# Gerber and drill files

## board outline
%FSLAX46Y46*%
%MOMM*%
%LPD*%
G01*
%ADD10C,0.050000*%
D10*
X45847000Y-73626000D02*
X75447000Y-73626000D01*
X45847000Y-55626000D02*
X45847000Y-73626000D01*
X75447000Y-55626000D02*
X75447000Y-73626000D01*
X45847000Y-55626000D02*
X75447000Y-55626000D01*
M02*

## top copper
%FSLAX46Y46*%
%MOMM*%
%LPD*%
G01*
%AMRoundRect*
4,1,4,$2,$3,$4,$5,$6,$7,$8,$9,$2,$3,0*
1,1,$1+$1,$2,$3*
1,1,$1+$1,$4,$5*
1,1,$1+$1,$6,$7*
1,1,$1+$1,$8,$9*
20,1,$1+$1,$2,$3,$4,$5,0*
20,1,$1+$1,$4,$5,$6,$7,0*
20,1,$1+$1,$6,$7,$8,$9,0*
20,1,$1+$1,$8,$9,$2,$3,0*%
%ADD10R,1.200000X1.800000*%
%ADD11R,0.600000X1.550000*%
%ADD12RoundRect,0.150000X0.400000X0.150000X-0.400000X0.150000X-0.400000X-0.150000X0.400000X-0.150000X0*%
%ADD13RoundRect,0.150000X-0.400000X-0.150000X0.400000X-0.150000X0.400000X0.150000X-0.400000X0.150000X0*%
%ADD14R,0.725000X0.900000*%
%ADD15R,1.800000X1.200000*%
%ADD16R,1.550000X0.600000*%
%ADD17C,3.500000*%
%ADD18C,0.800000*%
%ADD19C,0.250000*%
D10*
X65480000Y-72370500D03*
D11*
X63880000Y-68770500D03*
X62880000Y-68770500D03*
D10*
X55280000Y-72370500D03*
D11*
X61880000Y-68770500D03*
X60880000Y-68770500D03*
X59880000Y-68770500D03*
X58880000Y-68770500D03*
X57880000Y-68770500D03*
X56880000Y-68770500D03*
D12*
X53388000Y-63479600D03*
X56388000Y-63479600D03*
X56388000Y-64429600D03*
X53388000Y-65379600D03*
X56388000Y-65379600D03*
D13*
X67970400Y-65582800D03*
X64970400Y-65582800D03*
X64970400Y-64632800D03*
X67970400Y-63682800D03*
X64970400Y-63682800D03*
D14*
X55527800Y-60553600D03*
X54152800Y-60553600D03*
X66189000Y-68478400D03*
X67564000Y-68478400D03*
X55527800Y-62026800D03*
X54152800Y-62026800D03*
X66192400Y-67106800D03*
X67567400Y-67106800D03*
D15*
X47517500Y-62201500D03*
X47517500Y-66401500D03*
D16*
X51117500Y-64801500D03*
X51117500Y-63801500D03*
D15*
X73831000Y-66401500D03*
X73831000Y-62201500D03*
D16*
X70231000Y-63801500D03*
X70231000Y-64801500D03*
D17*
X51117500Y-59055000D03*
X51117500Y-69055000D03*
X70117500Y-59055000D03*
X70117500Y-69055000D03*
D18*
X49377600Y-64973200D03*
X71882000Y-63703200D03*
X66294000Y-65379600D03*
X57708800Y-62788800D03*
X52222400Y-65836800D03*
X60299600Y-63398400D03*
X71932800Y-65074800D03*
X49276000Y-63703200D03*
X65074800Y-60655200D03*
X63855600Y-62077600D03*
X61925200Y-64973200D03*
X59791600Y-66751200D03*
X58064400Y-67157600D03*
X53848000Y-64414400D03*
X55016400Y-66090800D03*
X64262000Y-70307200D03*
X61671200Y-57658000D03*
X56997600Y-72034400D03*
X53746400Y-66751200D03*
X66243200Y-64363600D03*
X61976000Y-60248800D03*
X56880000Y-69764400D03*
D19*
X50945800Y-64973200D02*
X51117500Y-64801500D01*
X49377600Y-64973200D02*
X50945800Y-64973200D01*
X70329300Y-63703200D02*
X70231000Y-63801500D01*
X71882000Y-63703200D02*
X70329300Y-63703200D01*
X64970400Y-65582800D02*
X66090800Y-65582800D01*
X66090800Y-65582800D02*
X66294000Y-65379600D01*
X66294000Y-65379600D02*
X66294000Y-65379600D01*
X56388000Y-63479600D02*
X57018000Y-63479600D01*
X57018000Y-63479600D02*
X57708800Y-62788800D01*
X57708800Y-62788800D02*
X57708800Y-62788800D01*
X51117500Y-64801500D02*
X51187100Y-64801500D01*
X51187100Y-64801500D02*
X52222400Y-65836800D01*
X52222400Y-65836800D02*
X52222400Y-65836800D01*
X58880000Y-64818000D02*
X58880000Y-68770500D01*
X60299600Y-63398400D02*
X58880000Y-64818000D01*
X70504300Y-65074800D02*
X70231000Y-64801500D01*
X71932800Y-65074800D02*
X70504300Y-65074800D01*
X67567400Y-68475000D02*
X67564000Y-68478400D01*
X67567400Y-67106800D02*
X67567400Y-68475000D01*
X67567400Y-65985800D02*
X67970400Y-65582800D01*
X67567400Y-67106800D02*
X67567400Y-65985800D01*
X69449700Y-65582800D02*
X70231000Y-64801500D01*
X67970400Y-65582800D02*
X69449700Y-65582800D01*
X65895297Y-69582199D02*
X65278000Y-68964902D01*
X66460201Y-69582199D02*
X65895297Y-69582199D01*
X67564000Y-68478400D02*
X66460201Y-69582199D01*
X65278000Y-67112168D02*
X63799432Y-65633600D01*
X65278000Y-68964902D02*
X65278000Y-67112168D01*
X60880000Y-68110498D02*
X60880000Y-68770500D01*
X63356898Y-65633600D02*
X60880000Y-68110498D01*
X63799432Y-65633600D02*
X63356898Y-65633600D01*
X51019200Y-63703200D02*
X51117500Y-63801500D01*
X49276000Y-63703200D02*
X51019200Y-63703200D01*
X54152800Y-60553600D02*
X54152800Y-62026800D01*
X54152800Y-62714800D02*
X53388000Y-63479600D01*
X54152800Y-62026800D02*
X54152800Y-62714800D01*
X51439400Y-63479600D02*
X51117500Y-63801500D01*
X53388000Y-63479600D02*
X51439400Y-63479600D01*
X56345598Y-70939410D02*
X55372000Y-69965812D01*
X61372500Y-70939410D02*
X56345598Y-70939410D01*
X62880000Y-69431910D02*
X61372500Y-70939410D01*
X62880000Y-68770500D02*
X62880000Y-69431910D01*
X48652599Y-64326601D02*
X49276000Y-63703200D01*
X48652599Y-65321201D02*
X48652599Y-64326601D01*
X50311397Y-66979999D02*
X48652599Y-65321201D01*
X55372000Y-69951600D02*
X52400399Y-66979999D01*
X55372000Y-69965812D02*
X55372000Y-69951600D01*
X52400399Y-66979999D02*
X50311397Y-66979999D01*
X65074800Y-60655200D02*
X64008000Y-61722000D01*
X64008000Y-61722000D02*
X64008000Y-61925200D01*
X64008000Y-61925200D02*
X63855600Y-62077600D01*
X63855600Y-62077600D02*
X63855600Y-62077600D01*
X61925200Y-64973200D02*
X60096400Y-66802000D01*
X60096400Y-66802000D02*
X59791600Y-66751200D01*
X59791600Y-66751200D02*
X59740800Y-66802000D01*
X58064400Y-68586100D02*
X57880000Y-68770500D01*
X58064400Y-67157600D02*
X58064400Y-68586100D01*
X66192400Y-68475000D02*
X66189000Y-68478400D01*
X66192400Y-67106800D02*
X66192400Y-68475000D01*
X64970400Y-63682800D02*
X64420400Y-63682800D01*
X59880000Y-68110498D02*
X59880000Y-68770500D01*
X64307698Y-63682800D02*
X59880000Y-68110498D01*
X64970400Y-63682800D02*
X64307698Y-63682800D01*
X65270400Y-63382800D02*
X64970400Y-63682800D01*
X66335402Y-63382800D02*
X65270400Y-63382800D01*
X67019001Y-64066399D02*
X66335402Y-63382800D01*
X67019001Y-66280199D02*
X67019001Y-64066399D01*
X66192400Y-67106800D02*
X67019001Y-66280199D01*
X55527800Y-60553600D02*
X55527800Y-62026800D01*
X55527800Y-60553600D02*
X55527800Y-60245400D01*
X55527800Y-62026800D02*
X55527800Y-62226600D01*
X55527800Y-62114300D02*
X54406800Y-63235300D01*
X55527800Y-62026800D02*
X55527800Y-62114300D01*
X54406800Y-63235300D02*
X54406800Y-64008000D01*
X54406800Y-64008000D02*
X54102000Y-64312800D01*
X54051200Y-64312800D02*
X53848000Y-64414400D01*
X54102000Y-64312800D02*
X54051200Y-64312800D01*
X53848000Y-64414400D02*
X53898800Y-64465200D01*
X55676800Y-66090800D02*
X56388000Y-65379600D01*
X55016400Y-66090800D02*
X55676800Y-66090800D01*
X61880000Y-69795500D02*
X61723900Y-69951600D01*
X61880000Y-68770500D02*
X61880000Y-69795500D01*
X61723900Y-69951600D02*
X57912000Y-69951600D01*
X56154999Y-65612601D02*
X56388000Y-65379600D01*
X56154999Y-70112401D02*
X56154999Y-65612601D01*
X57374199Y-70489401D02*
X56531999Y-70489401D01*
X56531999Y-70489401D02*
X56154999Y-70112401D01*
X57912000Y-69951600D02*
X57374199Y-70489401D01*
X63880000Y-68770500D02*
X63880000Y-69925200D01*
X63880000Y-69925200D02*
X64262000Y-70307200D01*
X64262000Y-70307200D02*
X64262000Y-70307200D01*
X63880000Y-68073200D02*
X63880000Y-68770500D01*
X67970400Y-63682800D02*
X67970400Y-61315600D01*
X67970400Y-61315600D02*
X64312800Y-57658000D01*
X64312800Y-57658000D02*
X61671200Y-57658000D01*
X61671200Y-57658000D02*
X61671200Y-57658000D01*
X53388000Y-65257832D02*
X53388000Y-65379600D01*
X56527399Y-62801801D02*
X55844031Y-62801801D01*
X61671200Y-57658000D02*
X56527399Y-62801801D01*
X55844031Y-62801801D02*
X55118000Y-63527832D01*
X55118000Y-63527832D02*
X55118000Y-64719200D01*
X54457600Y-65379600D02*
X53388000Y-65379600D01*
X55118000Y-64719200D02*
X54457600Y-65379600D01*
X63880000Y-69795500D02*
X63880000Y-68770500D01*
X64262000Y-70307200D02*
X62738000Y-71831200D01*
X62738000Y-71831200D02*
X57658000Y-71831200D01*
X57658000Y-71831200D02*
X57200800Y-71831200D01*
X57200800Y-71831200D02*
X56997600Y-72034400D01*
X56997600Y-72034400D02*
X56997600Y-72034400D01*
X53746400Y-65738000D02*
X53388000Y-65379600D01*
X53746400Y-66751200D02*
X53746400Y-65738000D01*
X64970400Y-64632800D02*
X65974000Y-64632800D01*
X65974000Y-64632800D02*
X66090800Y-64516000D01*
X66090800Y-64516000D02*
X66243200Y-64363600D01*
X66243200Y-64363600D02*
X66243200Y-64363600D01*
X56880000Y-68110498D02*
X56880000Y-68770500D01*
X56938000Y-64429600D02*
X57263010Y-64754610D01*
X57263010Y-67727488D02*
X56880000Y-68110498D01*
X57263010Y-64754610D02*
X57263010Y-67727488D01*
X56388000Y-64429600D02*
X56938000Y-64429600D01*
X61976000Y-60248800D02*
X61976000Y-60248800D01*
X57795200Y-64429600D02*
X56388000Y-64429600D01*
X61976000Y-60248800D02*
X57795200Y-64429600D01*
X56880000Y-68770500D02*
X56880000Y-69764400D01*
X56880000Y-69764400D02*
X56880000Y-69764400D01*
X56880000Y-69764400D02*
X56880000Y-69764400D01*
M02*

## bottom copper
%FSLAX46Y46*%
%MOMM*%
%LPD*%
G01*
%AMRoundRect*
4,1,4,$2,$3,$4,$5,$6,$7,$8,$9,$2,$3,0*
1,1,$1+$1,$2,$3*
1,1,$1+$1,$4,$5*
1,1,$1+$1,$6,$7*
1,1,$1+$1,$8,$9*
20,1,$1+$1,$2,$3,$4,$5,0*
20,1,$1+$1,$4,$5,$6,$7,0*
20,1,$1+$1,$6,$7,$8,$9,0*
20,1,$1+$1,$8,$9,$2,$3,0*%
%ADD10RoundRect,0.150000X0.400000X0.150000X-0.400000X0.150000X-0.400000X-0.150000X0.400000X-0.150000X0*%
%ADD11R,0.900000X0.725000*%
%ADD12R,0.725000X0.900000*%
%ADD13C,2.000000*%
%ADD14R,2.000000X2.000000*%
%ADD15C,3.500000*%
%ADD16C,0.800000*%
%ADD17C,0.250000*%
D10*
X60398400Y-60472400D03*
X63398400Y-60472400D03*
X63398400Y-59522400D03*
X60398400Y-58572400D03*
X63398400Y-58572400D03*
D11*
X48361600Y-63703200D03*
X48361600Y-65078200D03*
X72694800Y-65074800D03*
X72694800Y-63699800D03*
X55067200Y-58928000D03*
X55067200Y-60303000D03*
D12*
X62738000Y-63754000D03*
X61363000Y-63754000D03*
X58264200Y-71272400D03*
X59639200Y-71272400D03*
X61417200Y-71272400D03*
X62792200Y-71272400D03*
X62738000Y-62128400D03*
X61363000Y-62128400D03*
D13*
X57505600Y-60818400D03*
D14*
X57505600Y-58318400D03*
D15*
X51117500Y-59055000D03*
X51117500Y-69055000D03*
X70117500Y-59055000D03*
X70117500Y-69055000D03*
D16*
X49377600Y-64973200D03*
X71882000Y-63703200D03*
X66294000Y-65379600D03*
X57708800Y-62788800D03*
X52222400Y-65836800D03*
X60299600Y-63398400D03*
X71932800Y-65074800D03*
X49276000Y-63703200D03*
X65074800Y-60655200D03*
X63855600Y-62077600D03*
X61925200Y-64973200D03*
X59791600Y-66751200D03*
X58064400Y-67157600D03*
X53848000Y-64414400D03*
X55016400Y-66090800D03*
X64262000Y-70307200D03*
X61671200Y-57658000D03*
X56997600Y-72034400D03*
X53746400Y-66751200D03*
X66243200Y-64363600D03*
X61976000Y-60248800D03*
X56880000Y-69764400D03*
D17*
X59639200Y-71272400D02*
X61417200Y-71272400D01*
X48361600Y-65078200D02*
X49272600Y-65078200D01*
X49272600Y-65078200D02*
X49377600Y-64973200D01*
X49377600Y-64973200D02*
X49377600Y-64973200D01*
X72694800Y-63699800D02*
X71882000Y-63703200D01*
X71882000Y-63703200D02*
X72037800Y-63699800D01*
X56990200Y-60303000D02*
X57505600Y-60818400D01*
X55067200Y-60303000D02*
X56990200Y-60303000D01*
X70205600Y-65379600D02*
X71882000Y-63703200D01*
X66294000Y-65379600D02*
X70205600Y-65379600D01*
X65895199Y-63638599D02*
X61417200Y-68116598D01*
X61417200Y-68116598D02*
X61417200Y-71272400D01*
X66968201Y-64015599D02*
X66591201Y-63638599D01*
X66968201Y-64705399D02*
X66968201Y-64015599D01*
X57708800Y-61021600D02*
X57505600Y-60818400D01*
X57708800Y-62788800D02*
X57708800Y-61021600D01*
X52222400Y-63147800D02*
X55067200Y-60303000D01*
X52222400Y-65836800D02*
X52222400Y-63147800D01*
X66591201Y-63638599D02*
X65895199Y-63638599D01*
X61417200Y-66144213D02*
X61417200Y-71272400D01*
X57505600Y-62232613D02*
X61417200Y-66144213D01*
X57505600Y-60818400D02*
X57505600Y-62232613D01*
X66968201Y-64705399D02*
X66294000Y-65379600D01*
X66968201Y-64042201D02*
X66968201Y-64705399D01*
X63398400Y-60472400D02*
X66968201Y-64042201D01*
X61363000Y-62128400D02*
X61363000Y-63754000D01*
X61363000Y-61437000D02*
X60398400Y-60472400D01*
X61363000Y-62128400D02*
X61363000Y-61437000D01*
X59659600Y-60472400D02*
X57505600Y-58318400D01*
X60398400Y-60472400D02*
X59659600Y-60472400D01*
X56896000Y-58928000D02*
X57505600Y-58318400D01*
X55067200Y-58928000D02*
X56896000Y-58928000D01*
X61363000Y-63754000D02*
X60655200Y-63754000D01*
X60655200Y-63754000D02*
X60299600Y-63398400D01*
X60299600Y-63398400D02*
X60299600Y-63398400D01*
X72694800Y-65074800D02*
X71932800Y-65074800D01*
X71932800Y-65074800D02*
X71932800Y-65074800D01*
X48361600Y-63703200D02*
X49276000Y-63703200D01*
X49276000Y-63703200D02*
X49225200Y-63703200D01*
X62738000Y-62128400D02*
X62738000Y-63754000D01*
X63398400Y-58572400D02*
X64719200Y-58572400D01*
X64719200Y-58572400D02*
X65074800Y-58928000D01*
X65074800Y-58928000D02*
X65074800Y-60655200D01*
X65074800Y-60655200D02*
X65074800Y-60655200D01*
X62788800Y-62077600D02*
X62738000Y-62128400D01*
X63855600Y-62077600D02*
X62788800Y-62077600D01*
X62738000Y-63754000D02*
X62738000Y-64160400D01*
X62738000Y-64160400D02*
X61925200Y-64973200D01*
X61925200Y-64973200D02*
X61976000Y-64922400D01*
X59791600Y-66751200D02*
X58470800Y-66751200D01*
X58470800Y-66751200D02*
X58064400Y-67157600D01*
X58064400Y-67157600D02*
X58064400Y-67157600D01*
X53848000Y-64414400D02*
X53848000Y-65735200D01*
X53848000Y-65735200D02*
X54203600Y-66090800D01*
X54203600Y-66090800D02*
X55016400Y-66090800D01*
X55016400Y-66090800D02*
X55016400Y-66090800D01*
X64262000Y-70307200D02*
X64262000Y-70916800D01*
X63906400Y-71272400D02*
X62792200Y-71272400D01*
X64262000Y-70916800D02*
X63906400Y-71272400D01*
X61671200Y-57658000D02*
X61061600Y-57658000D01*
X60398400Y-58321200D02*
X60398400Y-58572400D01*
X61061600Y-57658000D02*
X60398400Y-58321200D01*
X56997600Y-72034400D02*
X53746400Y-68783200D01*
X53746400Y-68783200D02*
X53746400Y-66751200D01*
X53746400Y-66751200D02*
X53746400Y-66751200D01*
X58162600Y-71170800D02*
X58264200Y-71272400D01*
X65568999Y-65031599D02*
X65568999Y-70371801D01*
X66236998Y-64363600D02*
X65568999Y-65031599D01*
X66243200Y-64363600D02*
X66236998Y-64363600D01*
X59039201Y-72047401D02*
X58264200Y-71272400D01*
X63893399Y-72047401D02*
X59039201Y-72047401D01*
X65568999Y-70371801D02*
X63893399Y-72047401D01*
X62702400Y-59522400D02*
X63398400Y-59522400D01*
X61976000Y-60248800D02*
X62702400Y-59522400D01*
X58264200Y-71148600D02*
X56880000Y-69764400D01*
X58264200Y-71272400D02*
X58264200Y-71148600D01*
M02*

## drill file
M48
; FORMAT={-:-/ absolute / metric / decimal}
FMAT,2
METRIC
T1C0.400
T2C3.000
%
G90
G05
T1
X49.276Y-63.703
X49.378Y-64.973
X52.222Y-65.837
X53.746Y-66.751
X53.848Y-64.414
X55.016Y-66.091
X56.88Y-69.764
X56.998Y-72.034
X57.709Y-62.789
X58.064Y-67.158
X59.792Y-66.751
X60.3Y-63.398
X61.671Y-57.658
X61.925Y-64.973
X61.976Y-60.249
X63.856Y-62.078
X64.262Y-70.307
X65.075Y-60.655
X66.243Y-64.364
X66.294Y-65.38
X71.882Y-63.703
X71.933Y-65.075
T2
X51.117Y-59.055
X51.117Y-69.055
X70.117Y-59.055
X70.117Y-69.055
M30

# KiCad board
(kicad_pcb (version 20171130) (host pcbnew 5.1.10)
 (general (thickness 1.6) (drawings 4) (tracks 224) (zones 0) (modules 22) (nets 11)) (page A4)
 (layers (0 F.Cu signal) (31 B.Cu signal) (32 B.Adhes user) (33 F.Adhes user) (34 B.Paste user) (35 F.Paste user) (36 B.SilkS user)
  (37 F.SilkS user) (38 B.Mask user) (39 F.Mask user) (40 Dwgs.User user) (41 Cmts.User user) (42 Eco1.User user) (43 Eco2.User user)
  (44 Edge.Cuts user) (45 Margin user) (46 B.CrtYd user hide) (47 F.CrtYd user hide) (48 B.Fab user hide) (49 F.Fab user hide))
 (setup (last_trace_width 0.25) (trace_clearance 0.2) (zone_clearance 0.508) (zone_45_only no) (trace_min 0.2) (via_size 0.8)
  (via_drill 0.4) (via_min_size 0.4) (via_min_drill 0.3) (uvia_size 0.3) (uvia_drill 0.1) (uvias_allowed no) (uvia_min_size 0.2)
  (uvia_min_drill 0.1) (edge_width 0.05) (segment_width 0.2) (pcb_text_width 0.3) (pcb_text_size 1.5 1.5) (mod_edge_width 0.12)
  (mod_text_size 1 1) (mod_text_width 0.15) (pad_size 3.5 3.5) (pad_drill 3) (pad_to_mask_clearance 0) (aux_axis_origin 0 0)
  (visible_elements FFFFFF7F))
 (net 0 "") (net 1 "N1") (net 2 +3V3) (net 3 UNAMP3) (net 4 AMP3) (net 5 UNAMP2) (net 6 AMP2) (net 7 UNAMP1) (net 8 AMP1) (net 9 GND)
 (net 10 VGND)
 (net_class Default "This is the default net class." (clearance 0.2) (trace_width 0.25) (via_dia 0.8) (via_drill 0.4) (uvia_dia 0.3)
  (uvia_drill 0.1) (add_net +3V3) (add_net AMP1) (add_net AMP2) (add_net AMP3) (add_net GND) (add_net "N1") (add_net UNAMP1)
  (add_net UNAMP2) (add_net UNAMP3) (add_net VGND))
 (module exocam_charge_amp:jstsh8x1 (layer F.Cu) (at 59.69 66.2305)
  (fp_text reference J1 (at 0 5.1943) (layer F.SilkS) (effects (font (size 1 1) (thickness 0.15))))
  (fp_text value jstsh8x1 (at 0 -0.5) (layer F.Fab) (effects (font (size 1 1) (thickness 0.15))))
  (pad 9 smd rect (at 5.79 6.14) (size 1.2 1.8) (layers F.Cu F.Paste F.Mask) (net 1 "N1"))
  (pad 8 smd rect (at 4.19 2.54) (size 0.6 1.55) (layers F.Cu F.Paste F.Mask) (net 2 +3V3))
  (pad 7 smd rect (at 3.19 2.54) (size 0.6 1.55) (layers F.Cu F.Paste F.Mask) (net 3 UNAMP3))
  (pad 9 smd rect (at -4.41 6.14) (size 1.2 1.8) (layers F.Cu F.Paste F.Mask) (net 1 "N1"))
  (pad 6 smd rect (at 2.19 2.54) (size 0.6 1.55) (layers F.Cu F.Paste F.Mask) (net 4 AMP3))
  (pad 5 smd rect (at 1.19 2.54) (size 0.6 1.55) (layers F.Cu F.Paste F.Mask) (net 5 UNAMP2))
  (pad 4 smd rect (at 0.19 2.54) (size 0.6 1.55) (layers F.Cu F.Paste F.Mask) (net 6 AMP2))
  (pad 3 smd rect (at -0.81 2.54) (size 0.6 1.55) (layers F.Cu F.Paste F.Mask) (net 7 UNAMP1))
  (pad 2 smd rect (at -1.81 2.54) (size 0.6 1.55) (layers F.Cu F.Paste F.Mask) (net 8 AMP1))
  (pad 1 smd rect (at -2.81 2.54) (size 0.6 1.55) (layers F.Cu F.Paste F.Mask) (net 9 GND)))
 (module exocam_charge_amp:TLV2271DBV (layer F.Cu) (at 55.118 67.9196 180)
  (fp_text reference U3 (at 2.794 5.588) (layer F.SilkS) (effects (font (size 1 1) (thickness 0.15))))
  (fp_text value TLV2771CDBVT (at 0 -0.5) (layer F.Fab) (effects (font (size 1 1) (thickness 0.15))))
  (pad 4 smd roundrect (at 1.73 4.44 180) (size 1.1 0.6) (layers F.Cu F.Paste F.Mask) (roundrect_rratio 0.25) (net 3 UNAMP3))
  (pad 3 smd roundrect (at -1.27 4.44 180) (size 1.1 0.6) (layers F.Cu F.Paste F.Mask) (roundrect_rratio 0.25) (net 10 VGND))
  (pad 2 smd roundrect (at -1.27 3.49 180) (size 1.1 0.6) (layers F.Cu F.Paste F.Mask) (roundrect_rratio 0.25) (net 9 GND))
  (pad 5 smd roundrect (at 1.73 2.54 180) (size 1.1 0.6) (layers F.Cu F.Paste F.Mask) (roundrect_rratio 0.25) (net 2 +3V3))
  (pad 1 smd roundrect (at -1.27 2.54 180) (size 1.1 0.6) (layers F.Cu F.Paste F.Mask) (roundrect_rratio 0.25) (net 4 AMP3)))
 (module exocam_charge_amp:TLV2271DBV (layer F.Cu) (at 66.2404 61.1428)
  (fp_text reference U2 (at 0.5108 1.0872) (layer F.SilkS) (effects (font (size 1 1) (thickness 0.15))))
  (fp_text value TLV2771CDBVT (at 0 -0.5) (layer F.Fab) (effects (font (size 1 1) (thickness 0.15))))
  (pad 4 smd roundrect (at 1.73 4.44) (size 1.1 0.6) (layers F.Cu F.Paste F.Mask) (roundrect_rratio 0.25) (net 5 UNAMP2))
  (pad 3 smd roundrect (at -1.27 4.44) (size 1.1 0.6) (layers F.Cu F.Paste F.Mask) (roundrect_rratio 0.25) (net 10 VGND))
  (pad 2 smd roundrect (at -1.27 3.49) (size 1.1 0.6) (layers F.Cu F.Paste F.Mask) (roundrect_rratio 0.25) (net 9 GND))
  (pad 5 smd roundrect (at 1.73 2.54) (size 1.1 0.6) (layers F.Cu F.Paste F.Mask) (roundrect_rratio 0.25) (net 2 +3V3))
  (pad 1 smd roundrect (at -1.27 2.54) (size 1.1 0.6) (layers F.Cu F.Paste F.Mask) (roundrect_rratio 0.25) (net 6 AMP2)))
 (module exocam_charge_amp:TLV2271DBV (layer B.Cu) (at 62.1284 56.0324 180)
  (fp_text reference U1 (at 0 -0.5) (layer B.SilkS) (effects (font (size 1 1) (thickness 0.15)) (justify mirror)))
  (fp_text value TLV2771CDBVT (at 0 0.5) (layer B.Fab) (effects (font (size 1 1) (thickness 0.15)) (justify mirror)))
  (pad 4 smd roundrect (at 1.73 -4.44 180) (size 1.1 0.6) (layers B.Cu B.Paste B.Mask) (roundrect_rratio 0.25) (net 7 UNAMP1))
  (pad 3 smd roundrect (at -1.27 -4.44 180) (size 1.1 0.6) (layers B.Cu B.Paste B.Mask) (roundrect_rratio 0.25) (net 10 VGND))
  (pad 2 smd roundrect (at -1.27 -3.49 180) (size 1.1 0.6) (layers B.Cu B.Paste B.Mask) (roundrect_rratio 0.25) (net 9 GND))
  (pad 5 smd roundrect (at 1.73 -2.54 180) (size 1.1 0.6) (layers B.Cu B.Paste B.Mask) (roundrect_rratio 0.25) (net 2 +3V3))
  (pad 1 smd roundrect (at -1.27 -2.54 180) (size 1.1 0.6) (layers B.Cu B.Paste B.Mask) (roundrect_rratio 0.25) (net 8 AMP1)))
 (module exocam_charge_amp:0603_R (layer F.Cu) (at 55.4228 58.0136)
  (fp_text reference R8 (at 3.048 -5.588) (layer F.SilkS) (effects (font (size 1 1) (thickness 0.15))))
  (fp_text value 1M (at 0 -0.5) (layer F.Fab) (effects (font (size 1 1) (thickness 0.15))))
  (pad 2 smd rect (at 0.105 2.54) (size 0.725 0.9) (layers F.Cu F.Paste F.Mask) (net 4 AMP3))
  (pad 1 smd rect (at -1.27 2.54) (size 0.725 0.9) (layers F.Cu F.Paste F.Mask) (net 3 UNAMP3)))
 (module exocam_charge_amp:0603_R (layer B.Cu) (at 50.9016 63.8082 90)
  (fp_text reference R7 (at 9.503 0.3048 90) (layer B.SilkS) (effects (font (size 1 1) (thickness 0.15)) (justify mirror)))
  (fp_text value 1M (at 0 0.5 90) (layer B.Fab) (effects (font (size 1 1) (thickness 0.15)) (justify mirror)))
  (pad 2 smd rect (at 0.105 -2.54 90) (size 0.725 0.9) (layers B.Cu B.Paste B.Mask) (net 3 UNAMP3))
  (pad 1 smd rect (at -1.27 -2.54 90) (size 0.725 0.9) (layers B.Cu B.Paste B.Mask) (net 10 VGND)))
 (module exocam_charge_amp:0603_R (layer F.Cu) (at 66.294 71.0184 180)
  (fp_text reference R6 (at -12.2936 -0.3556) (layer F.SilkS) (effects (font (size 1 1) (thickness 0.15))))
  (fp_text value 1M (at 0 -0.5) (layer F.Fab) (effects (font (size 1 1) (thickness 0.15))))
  (pad 2 smd rect (at 0.105 2.54 180) (size 0.725 0.9) (layers F.Cu F.Paste F.Mask) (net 6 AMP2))
  (pad 1 smd rect (at -1.27 2.54 180) (size 0.725 0.9) (layers F.Cu F.Paste F.Mask) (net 5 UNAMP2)))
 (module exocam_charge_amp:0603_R (layer B.Cu) (at 70.1548 64.9698 270)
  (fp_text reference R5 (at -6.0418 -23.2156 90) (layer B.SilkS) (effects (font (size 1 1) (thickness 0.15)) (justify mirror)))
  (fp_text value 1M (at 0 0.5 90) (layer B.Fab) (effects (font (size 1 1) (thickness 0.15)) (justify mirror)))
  (pad 2 smd rect (at 0.105 -2.54 270) (size 0.725 0.9) (layers B.Cu B.Paste B.Mask) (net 5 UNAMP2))
  (pad 1 smd rect (at -1.27 -2.54 270) (size 0.725 0.9) (layers B.Cu B.Paste B.Mask) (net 10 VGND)))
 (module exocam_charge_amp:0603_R (layer B.Cu) (at 57.6072 59.033 90)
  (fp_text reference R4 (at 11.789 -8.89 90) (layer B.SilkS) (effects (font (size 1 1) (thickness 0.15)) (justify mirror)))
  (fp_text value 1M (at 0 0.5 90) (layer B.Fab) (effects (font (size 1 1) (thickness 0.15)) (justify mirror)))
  (pad 2 smd rect (at 0.105 -2.54 90) (size 0.725 0.9) (layers B.Cu B.Paste B.Mask) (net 7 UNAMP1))
  (pad 1 smd rect (at -1.27 -2.54 90) (size 0.725 0.9) (layers B.Cu B.Paste B.Mask) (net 10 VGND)))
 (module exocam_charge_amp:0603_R (layer B.Cu) (at 62.633 66.294)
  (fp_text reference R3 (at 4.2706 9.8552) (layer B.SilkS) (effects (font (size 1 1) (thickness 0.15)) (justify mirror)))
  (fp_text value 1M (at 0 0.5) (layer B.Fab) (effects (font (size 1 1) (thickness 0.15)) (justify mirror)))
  (pad 2 smd rect (at 0.105 -2.54) (size 0.725 0.9) (layers B.Cu B.Paste B.Mask) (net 8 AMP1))
  (pad 1 smd rect (at -1.27 -2.54) (size 0.725 0.9) (layers B.Cu B.Paste B.Mask) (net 7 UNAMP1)))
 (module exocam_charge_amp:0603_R (layer B.Cu) (at 58.3692 68.7324 180)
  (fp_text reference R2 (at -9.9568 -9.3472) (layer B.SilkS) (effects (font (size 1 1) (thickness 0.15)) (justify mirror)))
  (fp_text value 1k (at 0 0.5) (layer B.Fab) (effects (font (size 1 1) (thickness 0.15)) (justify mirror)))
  (pad 2 smd rect (at 0.105 -2.54 180) (size 0.725 0.9) (layers B.Cu B.Paste B.Mask) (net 9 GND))
  (pad 1 smd rect (at -1.27 -2.54 180) (size 0.725 0.9) (layers B.Cu B.Paste B.Mask) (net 10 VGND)))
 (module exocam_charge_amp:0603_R (layer B.Cu) (at 61.5222 68.7324 180)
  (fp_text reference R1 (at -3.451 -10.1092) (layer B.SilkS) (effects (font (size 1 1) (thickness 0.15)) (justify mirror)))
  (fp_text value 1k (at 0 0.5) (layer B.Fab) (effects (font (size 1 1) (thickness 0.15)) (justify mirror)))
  (pad 2 smd rect (at 0.105 -2.54 180) (size 0.725 0.9) (layers B.Cu B.Paste B.Mask) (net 10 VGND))
  (pad 1 smd rect (at -1.27 -2.54 180) (size 0.725 0.9) (layers B.Cu B.Paste B.Mask) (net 2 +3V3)))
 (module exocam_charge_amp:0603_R (layer F.Cu) (at 55.4228 59.4868)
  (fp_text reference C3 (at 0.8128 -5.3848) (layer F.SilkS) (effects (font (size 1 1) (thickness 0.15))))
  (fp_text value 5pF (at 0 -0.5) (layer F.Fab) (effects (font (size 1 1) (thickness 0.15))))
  (pad 2 smd rect (at 0.105 2.54) (size 0.725 0.9) (layers F.Cu F.Paste F.Mask) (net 4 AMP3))
  (pad 1 smd rect (at -1.27 2.54) (size 0.725 0.9) (layers F.Cu F.Paste F.Mask) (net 3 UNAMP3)))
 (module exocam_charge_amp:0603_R (layer F.Cu) (at 66.2974 69.6468 180)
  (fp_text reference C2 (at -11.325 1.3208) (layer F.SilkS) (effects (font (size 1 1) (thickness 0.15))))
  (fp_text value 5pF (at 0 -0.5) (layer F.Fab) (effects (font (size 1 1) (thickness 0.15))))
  (pad 2 smd rect (at 0.105 2.54 180) (size 0.725 0.9) (layers F.Cu F.Paste F.Mask) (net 6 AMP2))
  (pad 1 smd rect (at -1.27 2.54 180) (size 0.725 0.9) (layers F.Cu F.Paste F.Mask) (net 5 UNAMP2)))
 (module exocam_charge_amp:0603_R (layer B.Cu) (at 62.633 64.6684)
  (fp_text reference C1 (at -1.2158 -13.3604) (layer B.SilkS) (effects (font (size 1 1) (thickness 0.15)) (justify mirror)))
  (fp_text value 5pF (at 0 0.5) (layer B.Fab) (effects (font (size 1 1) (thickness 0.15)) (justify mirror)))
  (pad 2 smd rect (at 0.105 -2.54) (size 0.725 0.9) (layers B.Cu B.Paste B.Mask) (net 8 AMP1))
  (pad 1 smd rect (at -1.27 -2.54) (size 0.725 0.9) (layers B.Cu B.Paste B.Mask) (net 7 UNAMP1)))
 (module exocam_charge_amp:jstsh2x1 (layer F.Cu) (at 53.6575 66.6115 270)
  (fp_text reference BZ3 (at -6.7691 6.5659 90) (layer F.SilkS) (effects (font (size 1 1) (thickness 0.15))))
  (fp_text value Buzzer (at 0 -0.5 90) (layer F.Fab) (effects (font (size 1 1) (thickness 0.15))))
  (pad 3 smd rect (at -4.41 6.14 270) (size 1.2 1.8) (layers F.Cu F.Paste F.Mask))
  (pad 3 smd rect (at -0.21 6.14 270) (size 1.2 1.8) (layers F.Cu F.Paste F.Mask))
  (pad 2 smd rect (at -1.81 2.54 270) (size 0.6 1.55) (layers F.Cu F.Paste F.Mask) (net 10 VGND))
  (pad 1 smd rect (at -2.81 2.54 270) (size 0.6 1.55) (layers F.Cu F.Paste F.Mask) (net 3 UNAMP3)))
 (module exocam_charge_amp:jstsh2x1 (layer F.Cu) (at 67.691 61.9915 90)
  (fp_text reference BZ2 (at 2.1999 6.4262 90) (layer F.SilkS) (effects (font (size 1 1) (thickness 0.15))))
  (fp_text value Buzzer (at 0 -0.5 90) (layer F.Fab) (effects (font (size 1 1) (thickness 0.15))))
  (pad 3 smd rect (at -4.41 6.14 90) (size 1.2 1.8) (layers F.Cu F.Paste F.Mask))
  (pad 3 smd rect (at -0.21 6.14 90) (size 1.2 1.8) (layers F.Cu F.Paste F.Mask))
  (pad 2 smd rect (at -1.81 2.54 90) (size 0.6 1.55) (layers F.Cu F.Paste F.Mask) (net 10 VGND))
  (pad 1 smd rect (at -2.81 2.54 90) (size 0.6 1.55) (layers F.Cu F.Paste F.Mask) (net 5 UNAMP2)))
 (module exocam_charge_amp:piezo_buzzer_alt (layer B.Cu) (at 54.9656 59.8584 270)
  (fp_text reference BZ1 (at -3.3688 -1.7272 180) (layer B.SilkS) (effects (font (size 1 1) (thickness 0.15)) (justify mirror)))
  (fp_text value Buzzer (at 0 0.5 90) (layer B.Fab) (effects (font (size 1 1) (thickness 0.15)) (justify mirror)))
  (pad 2 smd circle (at 0.96 -2.54 270) (size 2 2) (layers B.Cu B.Paste B.Mask) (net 10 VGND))
  (pad 1 smd rect (at -1.54 -2.54 270) (size 2 2) (layers B.Cu B.Paste B.Mask) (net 7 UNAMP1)))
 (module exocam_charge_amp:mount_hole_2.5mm (layer F.Cu) (at 47.3075 57.785 90)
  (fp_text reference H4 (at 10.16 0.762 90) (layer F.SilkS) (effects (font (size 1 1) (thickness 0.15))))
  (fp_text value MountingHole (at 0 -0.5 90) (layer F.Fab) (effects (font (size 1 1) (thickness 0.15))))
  (pad 1 thru_hole circle (at -1.27 3.81 90) (size 3.5 3.5) (drill 3) (layers *.Cu *.Mask)))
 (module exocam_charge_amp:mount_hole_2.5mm (layer F.Cu) (at 47.3075 60.96 90)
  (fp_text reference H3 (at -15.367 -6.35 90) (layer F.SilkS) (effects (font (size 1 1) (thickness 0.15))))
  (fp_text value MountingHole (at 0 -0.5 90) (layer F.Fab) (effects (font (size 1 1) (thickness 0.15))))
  (pad 1 thru_hole circle (at -8.095 3.81 90) (size 3.5 3.5) (drill 3) (layers *.Cu *.Mask)))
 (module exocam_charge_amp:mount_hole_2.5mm (layer F.Cu) (at 66.1035 57.501 90)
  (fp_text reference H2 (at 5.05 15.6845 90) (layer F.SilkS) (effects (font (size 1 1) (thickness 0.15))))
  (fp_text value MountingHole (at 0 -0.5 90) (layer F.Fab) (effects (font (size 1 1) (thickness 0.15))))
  (pad 1 thru_hole circle (at -1.554 4.014 90) (size 3.5 3.5) (drill 3) (layers *.Cu *.Mask)))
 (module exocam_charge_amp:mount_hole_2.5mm (layer F.Cu) (at 66.1035 71.501 90)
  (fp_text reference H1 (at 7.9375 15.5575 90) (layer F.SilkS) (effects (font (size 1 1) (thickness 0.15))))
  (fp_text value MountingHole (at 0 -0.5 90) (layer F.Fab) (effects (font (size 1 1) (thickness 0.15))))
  (pad 1 thru_hole circle (at 2.446 4.014 90) (size 3.5 3.5) (drill 3) (layers *.Cu *.Mask)))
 (gr_line (start 45.847 73.626) (end 75.447 73.626) (layer Edge.Cuts) (width 0.05))
 (gr_line (start 45.847 55.626) (end 45.847 73.626) (layer Edge.Cuts) (width 0.05))
 (gr_line (start 75.447 55.626) (end 75.447 73.626) (layer Edge.Cuts) (width 0.05))
 (gr_line (start 45.847 55.626) (end 75.447 55.626) (layer Edge.Cuts) (width 0.05))
 (segment (start 59.6392 71.2724) (end 61.4172 71.2724) (width 0.25) (layer B.Cu) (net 10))
 (segment (start 48.3616 65.0782) (end 49.2726 65.0782) (width 0.25) (layer B.Cu) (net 10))
 (segment (start 49.2726 65.0782) (end 49.3776 64.9732) (width 0.25) (layer B.Cu) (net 10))
 (segment (start 49.3776 64.9732) (end 49.3776 64.9732) (width 0.25) (layer B.Cu) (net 10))
 (via (at 49.3776 64.9732) (size 0.8) (drill 0.4) (layers F.Cu B.Cu) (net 10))
 (segment (start 50.9458 64.9732) (end 51.1175 64.8015) (width 0.25) (layer F.Cu) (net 10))
 (segment (start 49.3776 64.9732) (end 50.9458 64.9732) (width 0.25) (layer F.Cu) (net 10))
 (segment (start 72.6948 63.6998) (end 71.882 63.7032) (width 0.25) (layer B.Cu) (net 10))
 (segment (start 71.882 63.7032) (end 72.0378 63.6998) (width 0.25) (layer B.Cu) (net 10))
 (via (at 71.882 63.7032) (size 0.8) (drill 0.4) (layers F.Cu B.Cu) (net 10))
 (segment (start 70.3293 63.7032) (end 70.231 63.8015) (width 0.25) (layer F.Cu) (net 10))
 (segment (start 71.882 63.7032) (end 70.3293 63.7032) (width 0.25) (layer F.Cu) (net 10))
 (segment (start 56.9902 60.303) (end 57.5056 60.8184) (width 0.25) (layer B.Cu) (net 10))
 (segment (start 55.0672 60.303) (end 56.9902 60.303) (width 0.25) (layer B.Cu) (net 10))
 (segment (start 64.9704 65.5828) (end 66.0908 65.5828) (width 0.25) (layer F.Cu) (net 10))
 (segment (start 66.0908 65.5828) (end 66.294 65.3796) (width 0.25) (layer F.Cu) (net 10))
 (segment (start 66.294 65.3796) (end 66.294 65.3796) (width 0.25) (layer F.Cu) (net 10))
 (via (at 66.294 65.3796) (size 0.8) (drill 0.4) (layers F.Cu B.Cu) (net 10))
 (segment (start 70.2056 65.3796) (end 71.882 63.7032) (width 0.25) (layer B.Cu) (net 10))
 (segment (start 66.294 65.3796) (end 70.2056 65.3796) (width 0.25) (layer B.Cu) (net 10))
 (segment (start 65.895199 63.638599) (end 61.4172 68.116598) (width 0.25) (layer B.Cu) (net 10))
 (segment (start 61.4172 68.116598) (end 61.4172 71.2724) (width 0.25) (layer B.Cu) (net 10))
 (segment (start 66.968201 64.015599) (end 66.591201 63.638599) (width 0.25) (layer B.Cu) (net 10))
 (segment (start 66.968201 64.705399) (end 66.968201 64.015599) (width 0.25) (layer B.Cu) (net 10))
 (segment (start 56.388 63.4796) (end 57.018 63.4796) (width 0.25) (layer F.Cu) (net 10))
 (segment (start 57.018 63.4796) (end 57.7088 62.7888) (width 0.25) (layer F.Cu) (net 10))
 (segment (start 57.7088 62.7888) (end 57.7088 62.7888) (width 0.25) (layer F.Cu) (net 10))
 (via (at 57.7088 62.7888) (size 0.8) (drill 0.4) (layers F.Cu B.Cu) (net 10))
 (segment (start 57.7088 61.0216) (end 57.5056 60.8184) (width 0.25) (layer B.Cu) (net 10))
 (segment (start 57.7088 62.7888) (end 57.7088 61.0216) (width 0.25) (layer B.Cu) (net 10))
 (segment (start 51.1175 64.8015) (end 51.1871 64.8015) (width 0.25) (layer F.Cu) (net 10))
 (segment (start 51.1871 64.8015) (end 52.2224 65.8368) (width 0.25) (layer F.Cu) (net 10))
 (segment (start 52.2224 65.8368) (end 52.2224 65.8368) (width 0.25) (layer F.Cu) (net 10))
 (via (at 52.2224 65.8368) (size 0.8) (drill 0.4) (layers F.Cu B.Cu) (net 10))
 (segment (start 52.2224 63.1478) (end 55.0672 60.303) (width 0.25) (layer B.Cu) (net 10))
 (segment (start 52.2224 65.8368) (end 52.2224 63.1478) (width 0.25) (layer B.Cu) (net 10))
 (segment (start 66.591201 63.638599) (end 65.895199 63.638599) (width 0.25) (layer B.Cu) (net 10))
 (segment (start 61.4172 66.144213) (end 61.4172 71.2724) (width 0.25) (layer B.Cu) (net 10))
 (segment (start 57.5056 62.232613) (end 61.4172 66.144213) (width 0.25) (layer B.Cu) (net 10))
 (segment (start 57.5056 60.8184) (end 57.5056 62.232613) (width 0.25) (layer B.Cu) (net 10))
 (segment (start 66.968201 64.705399) (end 66.294 65.3796) (width 0.25) (layer B.Cu) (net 10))
 (segment (start 66.968201 64.042201) (end 66.968201 64.705399) (width 0.25) (layer B.Cu) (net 10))
 (segment (start 63.3984 60.4724) (end 66.968201 64.042201) (width 0.25) (layer B.Cu) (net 10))
 (segment (start 61.363 62.1284) (end 61.363 63.754) (width 0.25) (layer B.Cu) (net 7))
 (segment (start 61.363 61.437) (end 60.3984 60.4724) (width 0.25) (layer B.Cu) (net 7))
 (segment (start 61.363 62.1284) (end 61.363 61.437) (width 0.25) (layer B.Cu) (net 7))
 (segment (start 59.6596 60.4724) (end 57.5056 58.3184) (width 0.25) (layer B.Cu) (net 7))
 (segment (start 60.3984 60.4724) (end 59.6596 60.4724) (width 0.25) (layer B.Cu) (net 7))
 (segment (start 56.896 58.928) (end 57.5056 58.3184) (width 0.25) (layer B.Cu) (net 7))
 (segment (start 55.0672 58.928) (end 56.896 58.928) (width 0.25) (layer B.Cu) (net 7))
 (segment (start 61.363 63.754) (end 60.6552 63.754) (width 0.25) (layer B.Cu) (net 7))
 (segment (start 60.6552 63.754) (end 60.2996 63.3984) (width 0.25) (layer B.Cu) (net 7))
 (segment (start 60.2996 63.3984) (end 60.2996 63.3984) (width 0.25) (layer B.Cu) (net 7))
 (via (at 60.2996 63.3984) (size 0.8) (drill 0.4) (layers F.Cu B.Cu) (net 7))
 (segment (start 58.88 64.818) (end 58.88 68.7705) (width 0.25) (layer F.Cu) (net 7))
 (segment (start 60.2996 63.3984) (end 58.88 64.818) (width 0.25) (layer F.Cu) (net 7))
 (segment (start 72.6948 65.0748) (end 71.9328 65.0748) (width 0.25) (layer B.Cu) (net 5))
 (segment (start 71.9328 65.0748) (end 71.9328 65.0748) (width 0.25) (layer B.Cu) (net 5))
 (via (at 71.9328 65.0748) (size 0.8) (drill 0.4) (layers F.Cu B.Cu) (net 5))
 (segment (start 70.5043 65.0748) (end 70.231 64.8015) (width 0.25) (layer F.Cu) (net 5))
 (segment (start 71.9328 65.0748) (end 70.5043 65.0748) (width 0.25) (layer F.Cu) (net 5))
 (segment (start 67.5674 68.475) (end 67.564 68.4784) (width 0.25) (layer F.Cu) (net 5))
 (segment (start 67.5674 67.1068) (end 67.5674 68.475) (width 0.25) (layer F.Cu) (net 5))
 (segment (start 67.5674 65.9858) (end 67.9704 65.5828) (width 0.25) (layer F.Cu) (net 5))
 (segment (start 67.5674 67.1068) (end 67.5674 65.9858) (width 0.25) (layer F.Cu) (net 5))
 (segment (start 69.4497 65.5828) (end 70.231 64.8015) (width 0.25) (layer F.Cu) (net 5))
 (segment (start 67.9704 65.5828) (end 69.4497 65.5828) (width 0.25) (layer F.Cu) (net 5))
 (segment (start 65.895297 69.582199) (end 65.278 68.964902) (width 0.25) (layer F.Cu) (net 5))
 (segment (start 66.460201 69.582199) (end 65.895297 69.582199) (width 0.25) (layer F.Cu) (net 5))
 (segment (start 67.564 68.4784) (end 66.460201 69.582199) (width 0.25) (layer F.Cu) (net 5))
 (segment (start 65.278 67.112168) (end 63.799432 65.6336) (width 0.25) (layer F.Cu) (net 5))
 (segment (start 65.278 68.964902) (end 65.278 67.112168) (width 0.25) (layer F.Cu) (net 5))
 (segment (start 60.88 68.110498) (end 60.88 68.7705) (width 0.25) (layer F.Cu) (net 5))
 (segment (start 63.356898 65.6336) (end 60.88 68.110498) (width 0.25) (layer F.Cu) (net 5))
 (segment (start 63.799432 65.6336) (end 63.356898 65.6336) (width 0.25) (layer F.Cu) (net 5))
 (segment (start 48.3616 63.7032) (end 49.276 63.7032) (width 0.25) (layer B.Cu) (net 3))
 (segment (start 49.276 63.7032) (end 49.2252 63.7032) (width 0.25) (layer B.Cu) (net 3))
 (via (at 49.276 63.7032) (size 0.8) (drill 0.4) (layers F.Cu B.Cu) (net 3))
 (segment (start 51.0192 63.7032) (end 51.1175 63.8015) (width 0.25) (layer F.Cu) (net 3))
 (segment (start 49.276 63.7032) (end 51.0192 63.7032) (width 0.25) (layer F.Cu) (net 3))
 (segment (start 54.1528 60.5536) (end 54.1528 62.0268) (width 0.25) (layer F.Cu) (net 3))
 (segment (start 54.1528 62.7148) (end 53.388 63.4796) (width 0.25) (layer F.Cu) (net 3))
 (segment (start 54.1528 62.0268) (end 54.1528 62.7148) (width 0.25) (layer F.Cu) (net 3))
 (segment (start 51.4394 63.4796) (end 51.1175 63.8015) (width 0.25) (layer F.Cu) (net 3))
 (segment (start 53.388 63.4796) (end 51.4394 63.4796) (width 0.25) (layer F.Cu) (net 3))
 (segment (start 56.345598 70.93941) (end 55.372 69.965812) (width 0.25) (layer F.Cu) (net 3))
 (segment (start 61.3725 70.93941) (end 56.345598 70.93941) (width 0.25) (layer F.Cu) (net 3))
 (segment (start 62.88 69.43191) (end 61.3725 70.93941) (width 0.25) (layer F.Cu) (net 3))
 (segment (start 62.88 68.7705) (end 62.88 69.43191) (width 0.25) (layer F.Cu) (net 3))
 (segment (start 48.652599 64.326601) (end 49.276 63.7032) (width 0.25) (layer F.Cu) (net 3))
 (segment (start 48.652599 65.321201) (end 48.652599 64.326601) (width 0.25) (layer F.Cu) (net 3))
 (segment (start 50.311397 66.979999) (end 48.652599 65.321201) (width 0.25) (layer F.Cu) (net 3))
 (segment (start 55.372 69.9516) (end 52.400399 66.979999) (width 0.25) (layer F.Cu) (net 3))
 (segment (start 55.372 69.965812) (end 55.372 69.9516) (width 0.25) (layer F.Cu) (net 3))
 (segment (start 52.400399 66.979999) (end 50.311397 66.979999) (width 0.25) (layer F.Cu) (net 3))
 (segment (start 62.738 62.1284) (end 62.738 63.754) (width 0.25) (layer B.Cu) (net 8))
 (segment (start 63.3984 58.5724) (end 64.7192 58.5724) (width 0.25) (layer B.Cu) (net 8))
 (segment (start 64.7192 58.5724) (end 65.0748 58.928) (width 0.25) (layer B.Cu) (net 8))
 (segment (start 65.0748 58.928) (end 65.0748 60.6552) (width 0.25) (layer B.Cu) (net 8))
 (segment (start 65.0748 60.6552) (end 65.0748 60.6552) (width 0.25) (layer B.Cu) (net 8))
 (via (at 65.0748 60.6552) (size 0.8) (drill 0.4) (layers F.Cu B.Cu) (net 8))
 (segment (start 65.0748 60.6552) (end 64.008 61.722) (width 0.25) (layer F.Cu) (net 8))
 (segment (start 64.008 61.722) (end 64.008 61.9252) (width 0.25) (layer F.Cu) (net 8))
 (segment (start 64.008 61.9252) (end 63.8556 62.0776) (width 0.25) (layer F.Cu) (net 8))
 (segment (start 63.8556 62.0776) (end 63.8556 62.0776) (width 0.25) (layer F.Cu) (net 8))
 (via (at 63.8556 62.0776) (size 0.8) (drill 0.4) (layers F.Cu B.Cu) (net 8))
 (segment (start 62.7888 62.0776) (end 62.738 62.1284) (width 0.25) (layer B.Cu) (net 8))
 (segment (start 63.8556 62.0776) (end 62.7888 62.0776) (width 0.25) (layer B.Cu) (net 8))
 (segment (start 62.738 63.754) (end 62.738 64.1604) (width 0.25) (layer B.Cu) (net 8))
 (segment (start 62.738 64.1604) (end 61.9252 64.9732) (width 0.25) (layer B.Cu) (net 8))
 (segment (start 61.9252 64.9732) (end 61.976 64.9224) (width 0.25) (layer B.Cu) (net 8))
 (via (at 61.9252 64.9732) (size 0.8) (drill 0.4) (layers F.Cu B.Cu) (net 8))
 (segment (start 61.9252 64.9732) (end 60.0964 66.802) (width 0.25) (layer F.Cu) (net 8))
 (segment (start 60.0964 66.802) (end 59.7916 66.7512) (width 0.25) (layer F.Cu) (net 8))
 (segment (start 59.7916 66.7512) (end 59.7408 66.802) (width 0.25) (layer F.Cu) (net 8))
 (via (at 59.7916 66.7512) (size 0.8) (drill 0.4) (layers F.Cu B.Cu) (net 8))
 (segment (start 59.7916 66.7512) (end 58.4708 66.7512) (width 0.25) (layer B.Cu) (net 8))
 (segment (start 58.4708 66.7512) (end 58.0644 67.1576) (width 0.25) (layer B.Cu) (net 8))
 (segment (start 58.0644 67.1576) (end 58.0644 67.1576) (width 0.25) (layer B.Cu) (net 8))
 (via (at 58.0644 67.1576) (size 0.8) (drill 0.4) (layers F.Cu B.Cu) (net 8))
 (segment (start 58.0644 68.5861) (end 57.88 68.7705) (width 0.25) (layer F.Cu) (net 8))
 (segment (start 58.0644 67.1576) (end 58.0644 68.5861) (width 0.25) (layer F.Cu) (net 8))
 (segment (start 66.1924 68.475) (end 66.189 68.4784) (width 0.25) (layer F.Cu) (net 6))
 (segment (start 66.1924 67.1068) (end 66.1924 68.475) (width 0.25) (layer F.Cu) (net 6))
 (segment (start 64.9704 63.6828) (end 64.4204 63.6828) (width 0.25) (layer F.Cu) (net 6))
 (segment (start 59.88 68.110498) (end 59.88 68.7705) (width 0.25) (layer F.Cu) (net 6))
 (segment (start 64.307698 63.6828) (end 59.88 68.110498) (width 0.25) (layer F.Cu) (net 6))
 (segment (start 64.9704 63.6828) (end 64.307698 63.6828) (width 0.25) (layer F.Cu) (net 6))
 (segment (start 65.2704 63.3828) (end 64.9704 63.6828) (width 0.25) (layer F.Cu) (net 6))
 (segment (start 66.335402 63.3828) (end 65.2704 63.3828) (width 0.25) (layer F.Cu) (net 6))
 (segment (start 67.019001 64.066399) (end 66.335402 63.3828) (width 0.25) (layer F.Cu) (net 6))
 (segment (start 67.019001 66.280199) (end 67.019001 64.066399) (width 0.25) (layer F.Cu) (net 6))
 (segment (start 66.1924 67.1068) (end 67.019001 66.280199) (width 0.25) (layer F.Cu) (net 6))
 (segment (start 55.5278 60.5536) (end 55.5278 62.0268) (width 0.25) (layer F.Cu) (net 4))
 (segment (start 55.5278 60.5536) (end 55.5278 60.2454) (width 0.25) (layer F.Cu) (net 4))
 (segment (start 55.5278 62.0268) (end 55.5278 62.2266) (width 0.25) (layer F.Cu) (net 4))
 (segment (start 55.5278 62.1143) (end 54.4068 63.2353) (width 0.25) (layer F.Cu) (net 4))
 (segment (start 55.5278 62.0268) (end 55.5278 62.1143) (width 0.25) (layer F.Cu) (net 4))
 (segment (start 54.4068 63.2353) (end 54.4068 64.008) (width 0.25) (layer F.Cu) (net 4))
 (segment (start 54.4068 64.008) (end 54.102 64.3128) (width 0.25) (layer F.Cu) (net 4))
 (segment (start 54.0512 64.3128) (end 53.848 64.4144) (width 0.25) (layer F.Cu) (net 4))
 (segment (start 54.102 64.3128) (end 54.0512 64.3128) (width 0.25) (layer F.Cu) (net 4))
 (segment (start 53.848 64.4144) (end 53.8988 64.4652) (width 0.25) (layer F.Cu) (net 4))
 (via (at 53.848 64.4144) (size 0.8) (drill 0.4) (layers F.Cu B.Cu) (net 4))
 (segment (start 53.848 64.4144) (end 53.848 65.7352) (width 0.25) (layer B.Cu) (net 4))
 (segment (start 53.848 65.7352) (end 54.2036 66.0908) (width 0.25) (layer B.Cu) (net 4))
 (segment (start 54.2036 66.0908) (end 55.0164 66.0908) (width 0.25) (layer B.Cu) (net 4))
 (segment (start 55.0164 66.0908) (end 55.0164 66.0908) (width 0.25) (layer B.Cu) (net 4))
 (via (at 55.0164 66.0908) (size 0.8) (drill 0.4) (layers F.Cu B.Cu) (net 4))
 (segment (start 55.6768 66.0908) (end 56.388 65.3796) (width 0.25) (layer F.Cu) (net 4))
 (segment (start 55.0164 66.0908) (end 55.6768 66.0908) (width 0.25) (layer F.Cu) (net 4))
 (segment (start 61.88 69.7955) (end 61.7239 69.9516) (width 0.25) (layer F.Cu) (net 4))
 (segment (start 61.88 68.7705) (end 61.88 69.7955) (width 0.25) (layer F.Cu) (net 4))
 (segment (start 61.7239 69.9516) (end 57.912 69.9516) (width 0.25) (layer F.Cu) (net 4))
 (segment (start 56.154999 65.612601) (end 56.388 65.3796) (width 0.25) (layer F.Cu) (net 4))
 (segment (start 56.154999 70.112401) (end 56.154999 65.612601) (width 0.25) (layer F.Cu) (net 4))
 (segment (start 57.374199 70.489401) (end 56.531999 70.489401) (width 0.25) (layer F.Cu) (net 4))
 (segment (start 56.531999 70.489401) (end 56.154999 70.112401) (width 0.25) (layer F.Cu) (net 4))
 (segment (start 57.912 69.9516) (end 57.374199 70.489401) (width 0.25) (layer F.Cu) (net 4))
 (segment (start 63.88 68.7705) (end 63.88 69.9252) (width 0.25) (layer F.Cu) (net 2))
 (segment (start 63.88 69.9252) (end 64.262 70.3072) (width 0.25) (layer F.Cu) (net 2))
 (segment (start 64.262 70.3072) (end 64.262 70.3072) (width 0.25) (layer F.Cu) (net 2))
 (via (at 64.262 70.3072) (size 0.8) (drill 0.4) (layers F.Cu B.Cu) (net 2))
 (segment (start 64.262 70.3072) (end 64.262 70.9168) (width 0.25) (layer B.Cu) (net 2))
 (segment (start 63.9064 71.2724) (end 62.7922 71.2724) (width 0.25) (layer B.Cu) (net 2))
 (segment (start 64.262 70.9168) (end 63.9064 71.2724) (width 0.25) (layer B.Cu) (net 2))
 (segment (start 63.88 68.0732) (end 63.88 68.7705) (width 0.25) (layer F.Cu) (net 2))
 (segment (start 67.9704 63.6828) (end 67.9704 61.3156) (width 0.25) (layer F.Cu) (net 2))
 (segment (start 67.9704 61.3156) (end 64.3128 57.658) (width 0.25) (layer F.Cu) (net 2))
 (segment (start 64.3128 57.658) (end 61.6712 57.658) (width 0.25) (layer F.Cu) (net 2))
 (segment (start 61.6712 57.658) (end 61.6712 57.658) (width 0.25) (layer F.Cu) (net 2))
 (via (at 61.6712 57.658) (size 0.8) (drill 0.4) (layers F.Cu B.Cu) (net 2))
 (segment (start 53.388 65.257832) (end 53.388 65.3796) (width 0.25) (layer F.Cu) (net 2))
 (segment (start 56.527399 62.801801) (end 55.844031 62.801801) (width 0.25) (layer F.Cu) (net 2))
 (segment (start 61.6712 57.658) (end 56.527399 62.801801) (width 0.25) (layer F.Cu) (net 2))
 (segment (start 61.6712 57.658) (end 61.0616 57.658) (width 0.25) (layer B.Cu) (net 2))
 (segment (start 60.3984 58.3212) (end 60.3984 58.5724) (width 0.25) (layer B.Cu) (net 2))
 (segment (start 61.0616 57.658) (end 60.3984 58.3212) (width 0.25) (layer B.Cu) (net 2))
 (segment (start 55.844031 62.801801) (end 55.118 63.527832) (width 0.25) (layer F.Cu) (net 2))
 (segment (start 55.118 63.527832) (end 55.118 64.7192) (width 0.25) (layer F.Cu) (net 2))
 (segment (start 54.4576 65.3796) (end 53.388 65.3796) (width 0.25) (layer F.Cu) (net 2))
 (segment (start 55.118 64.7192) (end 54.4576 65.3796) (width 0.25) (layer F.Cu) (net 2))
 (segment (start 63.88 69.7955) (end 63.88 68.7705) (width 0.25) (layer F.Cu) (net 2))
 (segment (start 64.262 70.3072) (end 62.738 71.8312) (width 0.25) (layer F.Cu) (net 2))
 (segment (start 62.738 71.8312) (end 57.658 71.8312) (width 0.25) (layer F.Cu) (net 2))
 (segment (start 57.658 71.8312) (end 57.2008 71.8312) (width 0.25) (layer F.Cu) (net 2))
 (segment (start 57.2008 71.8312) (end 56.9976 72.0344) (width 0.25) (layer F.Cu) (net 2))
 (segment (start 56.9976 72.0344) (end 56.9976 72.0344) (width 0.25) (layer F.Cu) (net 2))
 (via (at 56.9976 72.0344) (size 0.8) (drill 0.4) (layers F.Cu B.Cu) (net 2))
 (segment (start 56.9976 72.0344) (end 53.7464 68.7832) (width 0.25) (layer B.Cu) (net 2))
 (segment (start 53.7464 68.7832) (end 53.7464 66.7512) (width 0.25) (layer B.Cu) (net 2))
 (segment (start 53.7464 66.7512) (end 53.7464 66.7512) (width 0.25) (layer B.Cu) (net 2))
 (via (at 53.7464 66.7512) (size 0.8) (drill 0.4) (layers F.Cu B.Cu) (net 2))
 (segment (start 53.7464 65.738) (end 53.388 65.3796) (width 0.25) (layer F.Cu) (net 2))
 (segment (start 53.7464 66.7512) (end 53.7464 65.738) (width 0.25) (layer F.Cu) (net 2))
 (segment (start 58.1626 71.1708) (end 58.2642 71.2724) (width 0.25) (layer B.Cu) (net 9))
 (segment (start 64.9704 64.6328) (end 65.974 64.6328) (width 0.25) (layer F.Cu) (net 9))
 (segment (start 65.974 64.6328) (end 66.0908 64.516) (width 0.25) (layer F.Cu) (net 9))
 (segment (start 66.0908 64.516) (end 66.2432 64.3636) (width 0.25) (layer F.Cu) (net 9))
 (segment (start 66.2432 64.3636) (end 66.2432 64.3636) (width 0.25) (layer F.Cu) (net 9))
 (via (at 66.2432 64.3636) (size 0.8) (drill 0.4) (layers F.Cu B.Cu) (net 9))
 (segment (start 65.568999 65.031599) (end 65.568999 70.371801) (width 0.25) (layer B.Cu) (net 9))
 (segment (start 66.236998 64.3636) (end 65.568999 65.031599) (width 0.25) (layer B.Cu) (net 9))
 (segment (start 66.2432 64.3636) (end 66.236998 64.3636) (width 0.25) (layer B.Cu) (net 9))
 (segment (start 59.039201 72.047401) (end 58.2642 71.2724) (width 0.25) (layer B.Cu) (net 9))
 (segment (start 63.893399 72.047401) (end 59.039201 72.047401) (width 0.25) (layer B.Cu) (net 9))
 (segment (start 65.568999 70.371801) (end 63.893399 72.047401) (width 0.25) (layer B.Cu) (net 9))
 (segment (start 56.88 68.110498) (end 56.88 68.7705) (width 0.25) (layer F.Cu) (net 9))
 (segment (start 56.938 64.4296) (end 57.26301 64.75461) (width 0.25) (layer F.Cu) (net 9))
 (segment (start 57.26301 67.727488) (end 56.88 68.110498) (width 0.25) (layer F.Cu) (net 9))
 (segment (start 57.26301 64.75461) (end 57.26301 67.727488) (width 0.25) (layer F.Cu) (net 9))
 (segment (start 56.388 64.4296) (end 56.938 64.4296) (width 0.25) (layer F.Cu) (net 9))
 (segment (start 61.976 60.2488) (end 61.976 60.2488) (width 0.25) (layer F.Cu) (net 9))
 (via (at 61.976 60.2488) (size 0.8) (drill 0.4) (layers F.Cu B.Cu) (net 9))
 (segment (start 62.7024 59.5224) (end 63.3984 59.5224) (width 0.25) (layer B.Cu) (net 9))
 (segment (start 61.976 60.2488) (end 62.7024 59.5224) (width 0.25) (layer B.Cu) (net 9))
 (segment (start 57.7952 64.4296) (end 56.388 64.4296) (width 0.25) (layer F.Cu) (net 9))
 (segment (start 61.976 60.2488) (end 57.7952 64.4296) (width 0.25) (layer F.Cu) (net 9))
 (segment (start 56.88 68.7705) (end 56.88 69.7644) (width 0.25) (layer F.Cu) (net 9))
 (segment (start 56.88 69.7644) (end 56.88 69.7644) (width 0.25) (layer F.Cu) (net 9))
 (segment (start 56.88 69.7644) (end 56.88 69.7644) (width 0.25) (layer F.Cu) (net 9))
 (via (at 56.88 69.7644) (size 0.8) (drill 0.4) (layers F.Cu B.Cu) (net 9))
 (segment (start 58.2642 71.1486) (end 56.88 69.7644) (width 0.25) (layer B.Cu) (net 9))
 (segment (start 58.2642 71.2724) (end 58.2642 71.1486) (width 0.25) (layer B.Cu) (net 9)))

